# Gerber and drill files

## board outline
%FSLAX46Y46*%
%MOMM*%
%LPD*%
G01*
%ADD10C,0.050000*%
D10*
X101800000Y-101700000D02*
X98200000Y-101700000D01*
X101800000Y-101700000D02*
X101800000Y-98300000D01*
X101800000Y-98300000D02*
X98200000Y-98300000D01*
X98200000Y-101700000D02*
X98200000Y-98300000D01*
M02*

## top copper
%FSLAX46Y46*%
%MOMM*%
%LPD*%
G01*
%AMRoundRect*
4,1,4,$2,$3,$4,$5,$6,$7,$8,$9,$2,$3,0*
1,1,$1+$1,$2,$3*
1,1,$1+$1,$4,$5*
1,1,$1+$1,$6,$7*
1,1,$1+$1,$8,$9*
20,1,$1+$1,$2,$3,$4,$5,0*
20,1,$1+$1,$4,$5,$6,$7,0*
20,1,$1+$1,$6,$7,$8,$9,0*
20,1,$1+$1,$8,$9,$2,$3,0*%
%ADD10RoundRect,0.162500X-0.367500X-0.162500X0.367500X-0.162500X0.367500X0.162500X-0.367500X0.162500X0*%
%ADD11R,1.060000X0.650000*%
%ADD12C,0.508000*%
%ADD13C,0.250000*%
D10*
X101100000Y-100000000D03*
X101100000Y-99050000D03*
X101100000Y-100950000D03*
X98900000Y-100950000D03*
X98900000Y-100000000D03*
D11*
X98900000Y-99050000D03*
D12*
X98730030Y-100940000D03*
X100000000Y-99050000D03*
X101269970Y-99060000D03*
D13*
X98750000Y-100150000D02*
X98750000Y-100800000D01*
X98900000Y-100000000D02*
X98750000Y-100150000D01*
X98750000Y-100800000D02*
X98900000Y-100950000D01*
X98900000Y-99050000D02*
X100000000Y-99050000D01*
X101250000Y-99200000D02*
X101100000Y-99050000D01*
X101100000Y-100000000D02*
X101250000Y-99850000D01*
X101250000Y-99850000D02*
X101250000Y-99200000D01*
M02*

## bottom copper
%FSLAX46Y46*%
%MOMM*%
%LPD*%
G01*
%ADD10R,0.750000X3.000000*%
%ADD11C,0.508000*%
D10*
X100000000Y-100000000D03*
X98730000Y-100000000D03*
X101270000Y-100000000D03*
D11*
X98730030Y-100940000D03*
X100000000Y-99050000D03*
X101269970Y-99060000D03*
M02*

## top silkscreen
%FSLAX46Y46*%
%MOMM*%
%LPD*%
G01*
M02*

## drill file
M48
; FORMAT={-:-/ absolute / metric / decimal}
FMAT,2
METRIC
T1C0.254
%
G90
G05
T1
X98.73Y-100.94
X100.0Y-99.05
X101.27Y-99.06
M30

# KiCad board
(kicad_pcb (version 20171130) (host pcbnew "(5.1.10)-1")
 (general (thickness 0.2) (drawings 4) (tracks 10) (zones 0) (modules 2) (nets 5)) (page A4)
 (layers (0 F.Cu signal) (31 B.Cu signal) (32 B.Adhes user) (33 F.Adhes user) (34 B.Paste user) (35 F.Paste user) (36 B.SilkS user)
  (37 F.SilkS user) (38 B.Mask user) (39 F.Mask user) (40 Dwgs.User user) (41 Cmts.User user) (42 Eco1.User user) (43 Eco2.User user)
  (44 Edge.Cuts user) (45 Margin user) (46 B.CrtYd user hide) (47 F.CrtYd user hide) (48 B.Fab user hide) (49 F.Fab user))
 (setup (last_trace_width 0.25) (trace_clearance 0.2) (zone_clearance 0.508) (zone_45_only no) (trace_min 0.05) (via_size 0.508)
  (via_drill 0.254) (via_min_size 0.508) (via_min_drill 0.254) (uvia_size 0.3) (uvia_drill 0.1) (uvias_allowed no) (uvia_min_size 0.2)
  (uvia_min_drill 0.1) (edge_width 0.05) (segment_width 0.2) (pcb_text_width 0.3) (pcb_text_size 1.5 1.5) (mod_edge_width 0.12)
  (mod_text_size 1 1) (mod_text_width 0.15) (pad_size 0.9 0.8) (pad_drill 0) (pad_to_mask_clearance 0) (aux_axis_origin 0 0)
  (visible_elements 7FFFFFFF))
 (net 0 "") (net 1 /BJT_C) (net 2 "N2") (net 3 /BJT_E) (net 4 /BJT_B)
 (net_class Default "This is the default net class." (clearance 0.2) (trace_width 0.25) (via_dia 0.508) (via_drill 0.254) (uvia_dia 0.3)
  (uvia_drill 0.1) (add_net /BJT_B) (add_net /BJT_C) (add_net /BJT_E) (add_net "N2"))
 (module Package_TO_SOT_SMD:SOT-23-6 (layer F.Cu) (at 100 100)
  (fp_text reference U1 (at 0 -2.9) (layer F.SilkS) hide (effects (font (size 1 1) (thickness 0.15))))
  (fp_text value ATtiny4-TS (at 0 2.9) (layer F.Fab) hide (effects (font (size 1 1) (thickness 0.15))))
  (pad 5 smd roundrect (at 1.1 0) (size 1.06 0.65) (layers F.Cu F.Paste F.Mask) (roundrect_rratio 0.25) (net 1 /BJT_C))
  (pad 6 smd roundrect (at 1.1 -0.95) (size 1.06 0.65) (layers F.Cu F.Paste F.Mask) (roundrect_rratio 0.25) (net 1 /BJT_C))
  (pad 4 smd roundrect (at 1.1 0.95) (size 1.06 0.65) (layers F.Cu F.Paste F.Mask) (roundrect_rratio 0.25) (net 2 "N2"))
  (pad 3 smd roundrect (at -1.1 0.95) (size 1.06 0.65) (layers F.Cu F.Paste F.Mask) (roundrect_rratio 0.25) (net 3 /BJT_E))
  (pad 2 smd roundrect (at -1.1 0) (size 1.06 0.65) (layers F.Cu F.Paste F.Mask) (roundrect_rratio 0.25) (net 3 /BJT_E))
  (pad 1 smd rect (at -1.1 -0.95) (size 1.06 0.65) (layers F.Cu F.Paste F.Mask) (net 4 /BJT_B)))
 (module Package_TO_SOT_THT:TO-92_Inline (layer B.Cu) (at 101.27 100 180)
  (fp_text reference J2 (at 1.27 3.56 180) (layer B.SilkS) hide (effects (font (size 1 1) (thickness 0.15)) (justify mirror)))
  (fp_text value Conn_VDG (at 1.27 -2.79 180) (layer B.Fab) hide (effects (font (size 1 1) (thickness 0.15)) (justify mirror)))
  (pad 2 smd rect (at 1.27 0 180) (size 0.75 3) (layers B.Cu B.Paste B.Mask) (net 4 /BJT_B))
  (pad 3 smd rect (at 2.54 0 180) (size 0.75 3) (layers B.Cu B.Paste B.Mask) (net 3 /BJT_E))
  (pad 1 smd rect (at 0 0 180) (size 0.75 3) (layers B.Cu B.Paste B.Mask) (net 1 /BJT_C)))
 (gr_line (start 101.8 101.7) (end 98.2 101.7) (layer Edge.Cuts) (width 0.05))
 (gr_line (start 101.8 101.7) (end 101.8 98.3) (layer Edge.Cuts) (width 0.05))
 (gr_line (start 101.8 98.3) (end 98.2 98.3) (layer Edge.Cuts) (width 0.05))
 (gr_line (start 98.2 101.7) (end 98.2 98.3) (layer Edge.Cuts) (width 0.05))
 (via (at 98.73003 100.94) (size 0.508) (drill 0.254) (layers F.Cu B.Cu) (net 3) (status 1000000))
 (segment (start 98.75 100.15) (end 98.75 100.8) (width 0.25) (layer F.Cu) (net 3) (status 1000000))
 (segment (start 98.9 100) (end 98.75 100.15) (width 0.25) (layer F.Cu) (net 3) (status 1000000))
 (segment (start 98.75 100.8) (end 98.9 100.95) (width 0.25) (layer F.Cu) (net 3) (status 1000000))
 (via (at 100 99.05) (size 0.508) (drill 0.254) (layers F.Cu B.Cu) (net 4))
 (segment (start 98.9 99.05) (end 100 99.05) (width 0.25) (layer F.Cu) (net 4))
 (segment (start 101.25 99.2) (end 101.1 99.05) (width 0.25) (layer F.Cu) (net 1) (status 1000000))
 (segment (start 101.1 100) (end 101.25 99.85) (width 0.25) (layer F.Cu) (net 1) (status 1000000))
 (via (at 101.26997 99.06) (size 0.508) (drill 0.254) (layers F.Cu B.Cu) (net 1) (status 1000000))
 (segment (start 101.25 99.85) (end 101.25 99.2) (width 0.25) (layer F.Cu) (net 1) (status 1000000)))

